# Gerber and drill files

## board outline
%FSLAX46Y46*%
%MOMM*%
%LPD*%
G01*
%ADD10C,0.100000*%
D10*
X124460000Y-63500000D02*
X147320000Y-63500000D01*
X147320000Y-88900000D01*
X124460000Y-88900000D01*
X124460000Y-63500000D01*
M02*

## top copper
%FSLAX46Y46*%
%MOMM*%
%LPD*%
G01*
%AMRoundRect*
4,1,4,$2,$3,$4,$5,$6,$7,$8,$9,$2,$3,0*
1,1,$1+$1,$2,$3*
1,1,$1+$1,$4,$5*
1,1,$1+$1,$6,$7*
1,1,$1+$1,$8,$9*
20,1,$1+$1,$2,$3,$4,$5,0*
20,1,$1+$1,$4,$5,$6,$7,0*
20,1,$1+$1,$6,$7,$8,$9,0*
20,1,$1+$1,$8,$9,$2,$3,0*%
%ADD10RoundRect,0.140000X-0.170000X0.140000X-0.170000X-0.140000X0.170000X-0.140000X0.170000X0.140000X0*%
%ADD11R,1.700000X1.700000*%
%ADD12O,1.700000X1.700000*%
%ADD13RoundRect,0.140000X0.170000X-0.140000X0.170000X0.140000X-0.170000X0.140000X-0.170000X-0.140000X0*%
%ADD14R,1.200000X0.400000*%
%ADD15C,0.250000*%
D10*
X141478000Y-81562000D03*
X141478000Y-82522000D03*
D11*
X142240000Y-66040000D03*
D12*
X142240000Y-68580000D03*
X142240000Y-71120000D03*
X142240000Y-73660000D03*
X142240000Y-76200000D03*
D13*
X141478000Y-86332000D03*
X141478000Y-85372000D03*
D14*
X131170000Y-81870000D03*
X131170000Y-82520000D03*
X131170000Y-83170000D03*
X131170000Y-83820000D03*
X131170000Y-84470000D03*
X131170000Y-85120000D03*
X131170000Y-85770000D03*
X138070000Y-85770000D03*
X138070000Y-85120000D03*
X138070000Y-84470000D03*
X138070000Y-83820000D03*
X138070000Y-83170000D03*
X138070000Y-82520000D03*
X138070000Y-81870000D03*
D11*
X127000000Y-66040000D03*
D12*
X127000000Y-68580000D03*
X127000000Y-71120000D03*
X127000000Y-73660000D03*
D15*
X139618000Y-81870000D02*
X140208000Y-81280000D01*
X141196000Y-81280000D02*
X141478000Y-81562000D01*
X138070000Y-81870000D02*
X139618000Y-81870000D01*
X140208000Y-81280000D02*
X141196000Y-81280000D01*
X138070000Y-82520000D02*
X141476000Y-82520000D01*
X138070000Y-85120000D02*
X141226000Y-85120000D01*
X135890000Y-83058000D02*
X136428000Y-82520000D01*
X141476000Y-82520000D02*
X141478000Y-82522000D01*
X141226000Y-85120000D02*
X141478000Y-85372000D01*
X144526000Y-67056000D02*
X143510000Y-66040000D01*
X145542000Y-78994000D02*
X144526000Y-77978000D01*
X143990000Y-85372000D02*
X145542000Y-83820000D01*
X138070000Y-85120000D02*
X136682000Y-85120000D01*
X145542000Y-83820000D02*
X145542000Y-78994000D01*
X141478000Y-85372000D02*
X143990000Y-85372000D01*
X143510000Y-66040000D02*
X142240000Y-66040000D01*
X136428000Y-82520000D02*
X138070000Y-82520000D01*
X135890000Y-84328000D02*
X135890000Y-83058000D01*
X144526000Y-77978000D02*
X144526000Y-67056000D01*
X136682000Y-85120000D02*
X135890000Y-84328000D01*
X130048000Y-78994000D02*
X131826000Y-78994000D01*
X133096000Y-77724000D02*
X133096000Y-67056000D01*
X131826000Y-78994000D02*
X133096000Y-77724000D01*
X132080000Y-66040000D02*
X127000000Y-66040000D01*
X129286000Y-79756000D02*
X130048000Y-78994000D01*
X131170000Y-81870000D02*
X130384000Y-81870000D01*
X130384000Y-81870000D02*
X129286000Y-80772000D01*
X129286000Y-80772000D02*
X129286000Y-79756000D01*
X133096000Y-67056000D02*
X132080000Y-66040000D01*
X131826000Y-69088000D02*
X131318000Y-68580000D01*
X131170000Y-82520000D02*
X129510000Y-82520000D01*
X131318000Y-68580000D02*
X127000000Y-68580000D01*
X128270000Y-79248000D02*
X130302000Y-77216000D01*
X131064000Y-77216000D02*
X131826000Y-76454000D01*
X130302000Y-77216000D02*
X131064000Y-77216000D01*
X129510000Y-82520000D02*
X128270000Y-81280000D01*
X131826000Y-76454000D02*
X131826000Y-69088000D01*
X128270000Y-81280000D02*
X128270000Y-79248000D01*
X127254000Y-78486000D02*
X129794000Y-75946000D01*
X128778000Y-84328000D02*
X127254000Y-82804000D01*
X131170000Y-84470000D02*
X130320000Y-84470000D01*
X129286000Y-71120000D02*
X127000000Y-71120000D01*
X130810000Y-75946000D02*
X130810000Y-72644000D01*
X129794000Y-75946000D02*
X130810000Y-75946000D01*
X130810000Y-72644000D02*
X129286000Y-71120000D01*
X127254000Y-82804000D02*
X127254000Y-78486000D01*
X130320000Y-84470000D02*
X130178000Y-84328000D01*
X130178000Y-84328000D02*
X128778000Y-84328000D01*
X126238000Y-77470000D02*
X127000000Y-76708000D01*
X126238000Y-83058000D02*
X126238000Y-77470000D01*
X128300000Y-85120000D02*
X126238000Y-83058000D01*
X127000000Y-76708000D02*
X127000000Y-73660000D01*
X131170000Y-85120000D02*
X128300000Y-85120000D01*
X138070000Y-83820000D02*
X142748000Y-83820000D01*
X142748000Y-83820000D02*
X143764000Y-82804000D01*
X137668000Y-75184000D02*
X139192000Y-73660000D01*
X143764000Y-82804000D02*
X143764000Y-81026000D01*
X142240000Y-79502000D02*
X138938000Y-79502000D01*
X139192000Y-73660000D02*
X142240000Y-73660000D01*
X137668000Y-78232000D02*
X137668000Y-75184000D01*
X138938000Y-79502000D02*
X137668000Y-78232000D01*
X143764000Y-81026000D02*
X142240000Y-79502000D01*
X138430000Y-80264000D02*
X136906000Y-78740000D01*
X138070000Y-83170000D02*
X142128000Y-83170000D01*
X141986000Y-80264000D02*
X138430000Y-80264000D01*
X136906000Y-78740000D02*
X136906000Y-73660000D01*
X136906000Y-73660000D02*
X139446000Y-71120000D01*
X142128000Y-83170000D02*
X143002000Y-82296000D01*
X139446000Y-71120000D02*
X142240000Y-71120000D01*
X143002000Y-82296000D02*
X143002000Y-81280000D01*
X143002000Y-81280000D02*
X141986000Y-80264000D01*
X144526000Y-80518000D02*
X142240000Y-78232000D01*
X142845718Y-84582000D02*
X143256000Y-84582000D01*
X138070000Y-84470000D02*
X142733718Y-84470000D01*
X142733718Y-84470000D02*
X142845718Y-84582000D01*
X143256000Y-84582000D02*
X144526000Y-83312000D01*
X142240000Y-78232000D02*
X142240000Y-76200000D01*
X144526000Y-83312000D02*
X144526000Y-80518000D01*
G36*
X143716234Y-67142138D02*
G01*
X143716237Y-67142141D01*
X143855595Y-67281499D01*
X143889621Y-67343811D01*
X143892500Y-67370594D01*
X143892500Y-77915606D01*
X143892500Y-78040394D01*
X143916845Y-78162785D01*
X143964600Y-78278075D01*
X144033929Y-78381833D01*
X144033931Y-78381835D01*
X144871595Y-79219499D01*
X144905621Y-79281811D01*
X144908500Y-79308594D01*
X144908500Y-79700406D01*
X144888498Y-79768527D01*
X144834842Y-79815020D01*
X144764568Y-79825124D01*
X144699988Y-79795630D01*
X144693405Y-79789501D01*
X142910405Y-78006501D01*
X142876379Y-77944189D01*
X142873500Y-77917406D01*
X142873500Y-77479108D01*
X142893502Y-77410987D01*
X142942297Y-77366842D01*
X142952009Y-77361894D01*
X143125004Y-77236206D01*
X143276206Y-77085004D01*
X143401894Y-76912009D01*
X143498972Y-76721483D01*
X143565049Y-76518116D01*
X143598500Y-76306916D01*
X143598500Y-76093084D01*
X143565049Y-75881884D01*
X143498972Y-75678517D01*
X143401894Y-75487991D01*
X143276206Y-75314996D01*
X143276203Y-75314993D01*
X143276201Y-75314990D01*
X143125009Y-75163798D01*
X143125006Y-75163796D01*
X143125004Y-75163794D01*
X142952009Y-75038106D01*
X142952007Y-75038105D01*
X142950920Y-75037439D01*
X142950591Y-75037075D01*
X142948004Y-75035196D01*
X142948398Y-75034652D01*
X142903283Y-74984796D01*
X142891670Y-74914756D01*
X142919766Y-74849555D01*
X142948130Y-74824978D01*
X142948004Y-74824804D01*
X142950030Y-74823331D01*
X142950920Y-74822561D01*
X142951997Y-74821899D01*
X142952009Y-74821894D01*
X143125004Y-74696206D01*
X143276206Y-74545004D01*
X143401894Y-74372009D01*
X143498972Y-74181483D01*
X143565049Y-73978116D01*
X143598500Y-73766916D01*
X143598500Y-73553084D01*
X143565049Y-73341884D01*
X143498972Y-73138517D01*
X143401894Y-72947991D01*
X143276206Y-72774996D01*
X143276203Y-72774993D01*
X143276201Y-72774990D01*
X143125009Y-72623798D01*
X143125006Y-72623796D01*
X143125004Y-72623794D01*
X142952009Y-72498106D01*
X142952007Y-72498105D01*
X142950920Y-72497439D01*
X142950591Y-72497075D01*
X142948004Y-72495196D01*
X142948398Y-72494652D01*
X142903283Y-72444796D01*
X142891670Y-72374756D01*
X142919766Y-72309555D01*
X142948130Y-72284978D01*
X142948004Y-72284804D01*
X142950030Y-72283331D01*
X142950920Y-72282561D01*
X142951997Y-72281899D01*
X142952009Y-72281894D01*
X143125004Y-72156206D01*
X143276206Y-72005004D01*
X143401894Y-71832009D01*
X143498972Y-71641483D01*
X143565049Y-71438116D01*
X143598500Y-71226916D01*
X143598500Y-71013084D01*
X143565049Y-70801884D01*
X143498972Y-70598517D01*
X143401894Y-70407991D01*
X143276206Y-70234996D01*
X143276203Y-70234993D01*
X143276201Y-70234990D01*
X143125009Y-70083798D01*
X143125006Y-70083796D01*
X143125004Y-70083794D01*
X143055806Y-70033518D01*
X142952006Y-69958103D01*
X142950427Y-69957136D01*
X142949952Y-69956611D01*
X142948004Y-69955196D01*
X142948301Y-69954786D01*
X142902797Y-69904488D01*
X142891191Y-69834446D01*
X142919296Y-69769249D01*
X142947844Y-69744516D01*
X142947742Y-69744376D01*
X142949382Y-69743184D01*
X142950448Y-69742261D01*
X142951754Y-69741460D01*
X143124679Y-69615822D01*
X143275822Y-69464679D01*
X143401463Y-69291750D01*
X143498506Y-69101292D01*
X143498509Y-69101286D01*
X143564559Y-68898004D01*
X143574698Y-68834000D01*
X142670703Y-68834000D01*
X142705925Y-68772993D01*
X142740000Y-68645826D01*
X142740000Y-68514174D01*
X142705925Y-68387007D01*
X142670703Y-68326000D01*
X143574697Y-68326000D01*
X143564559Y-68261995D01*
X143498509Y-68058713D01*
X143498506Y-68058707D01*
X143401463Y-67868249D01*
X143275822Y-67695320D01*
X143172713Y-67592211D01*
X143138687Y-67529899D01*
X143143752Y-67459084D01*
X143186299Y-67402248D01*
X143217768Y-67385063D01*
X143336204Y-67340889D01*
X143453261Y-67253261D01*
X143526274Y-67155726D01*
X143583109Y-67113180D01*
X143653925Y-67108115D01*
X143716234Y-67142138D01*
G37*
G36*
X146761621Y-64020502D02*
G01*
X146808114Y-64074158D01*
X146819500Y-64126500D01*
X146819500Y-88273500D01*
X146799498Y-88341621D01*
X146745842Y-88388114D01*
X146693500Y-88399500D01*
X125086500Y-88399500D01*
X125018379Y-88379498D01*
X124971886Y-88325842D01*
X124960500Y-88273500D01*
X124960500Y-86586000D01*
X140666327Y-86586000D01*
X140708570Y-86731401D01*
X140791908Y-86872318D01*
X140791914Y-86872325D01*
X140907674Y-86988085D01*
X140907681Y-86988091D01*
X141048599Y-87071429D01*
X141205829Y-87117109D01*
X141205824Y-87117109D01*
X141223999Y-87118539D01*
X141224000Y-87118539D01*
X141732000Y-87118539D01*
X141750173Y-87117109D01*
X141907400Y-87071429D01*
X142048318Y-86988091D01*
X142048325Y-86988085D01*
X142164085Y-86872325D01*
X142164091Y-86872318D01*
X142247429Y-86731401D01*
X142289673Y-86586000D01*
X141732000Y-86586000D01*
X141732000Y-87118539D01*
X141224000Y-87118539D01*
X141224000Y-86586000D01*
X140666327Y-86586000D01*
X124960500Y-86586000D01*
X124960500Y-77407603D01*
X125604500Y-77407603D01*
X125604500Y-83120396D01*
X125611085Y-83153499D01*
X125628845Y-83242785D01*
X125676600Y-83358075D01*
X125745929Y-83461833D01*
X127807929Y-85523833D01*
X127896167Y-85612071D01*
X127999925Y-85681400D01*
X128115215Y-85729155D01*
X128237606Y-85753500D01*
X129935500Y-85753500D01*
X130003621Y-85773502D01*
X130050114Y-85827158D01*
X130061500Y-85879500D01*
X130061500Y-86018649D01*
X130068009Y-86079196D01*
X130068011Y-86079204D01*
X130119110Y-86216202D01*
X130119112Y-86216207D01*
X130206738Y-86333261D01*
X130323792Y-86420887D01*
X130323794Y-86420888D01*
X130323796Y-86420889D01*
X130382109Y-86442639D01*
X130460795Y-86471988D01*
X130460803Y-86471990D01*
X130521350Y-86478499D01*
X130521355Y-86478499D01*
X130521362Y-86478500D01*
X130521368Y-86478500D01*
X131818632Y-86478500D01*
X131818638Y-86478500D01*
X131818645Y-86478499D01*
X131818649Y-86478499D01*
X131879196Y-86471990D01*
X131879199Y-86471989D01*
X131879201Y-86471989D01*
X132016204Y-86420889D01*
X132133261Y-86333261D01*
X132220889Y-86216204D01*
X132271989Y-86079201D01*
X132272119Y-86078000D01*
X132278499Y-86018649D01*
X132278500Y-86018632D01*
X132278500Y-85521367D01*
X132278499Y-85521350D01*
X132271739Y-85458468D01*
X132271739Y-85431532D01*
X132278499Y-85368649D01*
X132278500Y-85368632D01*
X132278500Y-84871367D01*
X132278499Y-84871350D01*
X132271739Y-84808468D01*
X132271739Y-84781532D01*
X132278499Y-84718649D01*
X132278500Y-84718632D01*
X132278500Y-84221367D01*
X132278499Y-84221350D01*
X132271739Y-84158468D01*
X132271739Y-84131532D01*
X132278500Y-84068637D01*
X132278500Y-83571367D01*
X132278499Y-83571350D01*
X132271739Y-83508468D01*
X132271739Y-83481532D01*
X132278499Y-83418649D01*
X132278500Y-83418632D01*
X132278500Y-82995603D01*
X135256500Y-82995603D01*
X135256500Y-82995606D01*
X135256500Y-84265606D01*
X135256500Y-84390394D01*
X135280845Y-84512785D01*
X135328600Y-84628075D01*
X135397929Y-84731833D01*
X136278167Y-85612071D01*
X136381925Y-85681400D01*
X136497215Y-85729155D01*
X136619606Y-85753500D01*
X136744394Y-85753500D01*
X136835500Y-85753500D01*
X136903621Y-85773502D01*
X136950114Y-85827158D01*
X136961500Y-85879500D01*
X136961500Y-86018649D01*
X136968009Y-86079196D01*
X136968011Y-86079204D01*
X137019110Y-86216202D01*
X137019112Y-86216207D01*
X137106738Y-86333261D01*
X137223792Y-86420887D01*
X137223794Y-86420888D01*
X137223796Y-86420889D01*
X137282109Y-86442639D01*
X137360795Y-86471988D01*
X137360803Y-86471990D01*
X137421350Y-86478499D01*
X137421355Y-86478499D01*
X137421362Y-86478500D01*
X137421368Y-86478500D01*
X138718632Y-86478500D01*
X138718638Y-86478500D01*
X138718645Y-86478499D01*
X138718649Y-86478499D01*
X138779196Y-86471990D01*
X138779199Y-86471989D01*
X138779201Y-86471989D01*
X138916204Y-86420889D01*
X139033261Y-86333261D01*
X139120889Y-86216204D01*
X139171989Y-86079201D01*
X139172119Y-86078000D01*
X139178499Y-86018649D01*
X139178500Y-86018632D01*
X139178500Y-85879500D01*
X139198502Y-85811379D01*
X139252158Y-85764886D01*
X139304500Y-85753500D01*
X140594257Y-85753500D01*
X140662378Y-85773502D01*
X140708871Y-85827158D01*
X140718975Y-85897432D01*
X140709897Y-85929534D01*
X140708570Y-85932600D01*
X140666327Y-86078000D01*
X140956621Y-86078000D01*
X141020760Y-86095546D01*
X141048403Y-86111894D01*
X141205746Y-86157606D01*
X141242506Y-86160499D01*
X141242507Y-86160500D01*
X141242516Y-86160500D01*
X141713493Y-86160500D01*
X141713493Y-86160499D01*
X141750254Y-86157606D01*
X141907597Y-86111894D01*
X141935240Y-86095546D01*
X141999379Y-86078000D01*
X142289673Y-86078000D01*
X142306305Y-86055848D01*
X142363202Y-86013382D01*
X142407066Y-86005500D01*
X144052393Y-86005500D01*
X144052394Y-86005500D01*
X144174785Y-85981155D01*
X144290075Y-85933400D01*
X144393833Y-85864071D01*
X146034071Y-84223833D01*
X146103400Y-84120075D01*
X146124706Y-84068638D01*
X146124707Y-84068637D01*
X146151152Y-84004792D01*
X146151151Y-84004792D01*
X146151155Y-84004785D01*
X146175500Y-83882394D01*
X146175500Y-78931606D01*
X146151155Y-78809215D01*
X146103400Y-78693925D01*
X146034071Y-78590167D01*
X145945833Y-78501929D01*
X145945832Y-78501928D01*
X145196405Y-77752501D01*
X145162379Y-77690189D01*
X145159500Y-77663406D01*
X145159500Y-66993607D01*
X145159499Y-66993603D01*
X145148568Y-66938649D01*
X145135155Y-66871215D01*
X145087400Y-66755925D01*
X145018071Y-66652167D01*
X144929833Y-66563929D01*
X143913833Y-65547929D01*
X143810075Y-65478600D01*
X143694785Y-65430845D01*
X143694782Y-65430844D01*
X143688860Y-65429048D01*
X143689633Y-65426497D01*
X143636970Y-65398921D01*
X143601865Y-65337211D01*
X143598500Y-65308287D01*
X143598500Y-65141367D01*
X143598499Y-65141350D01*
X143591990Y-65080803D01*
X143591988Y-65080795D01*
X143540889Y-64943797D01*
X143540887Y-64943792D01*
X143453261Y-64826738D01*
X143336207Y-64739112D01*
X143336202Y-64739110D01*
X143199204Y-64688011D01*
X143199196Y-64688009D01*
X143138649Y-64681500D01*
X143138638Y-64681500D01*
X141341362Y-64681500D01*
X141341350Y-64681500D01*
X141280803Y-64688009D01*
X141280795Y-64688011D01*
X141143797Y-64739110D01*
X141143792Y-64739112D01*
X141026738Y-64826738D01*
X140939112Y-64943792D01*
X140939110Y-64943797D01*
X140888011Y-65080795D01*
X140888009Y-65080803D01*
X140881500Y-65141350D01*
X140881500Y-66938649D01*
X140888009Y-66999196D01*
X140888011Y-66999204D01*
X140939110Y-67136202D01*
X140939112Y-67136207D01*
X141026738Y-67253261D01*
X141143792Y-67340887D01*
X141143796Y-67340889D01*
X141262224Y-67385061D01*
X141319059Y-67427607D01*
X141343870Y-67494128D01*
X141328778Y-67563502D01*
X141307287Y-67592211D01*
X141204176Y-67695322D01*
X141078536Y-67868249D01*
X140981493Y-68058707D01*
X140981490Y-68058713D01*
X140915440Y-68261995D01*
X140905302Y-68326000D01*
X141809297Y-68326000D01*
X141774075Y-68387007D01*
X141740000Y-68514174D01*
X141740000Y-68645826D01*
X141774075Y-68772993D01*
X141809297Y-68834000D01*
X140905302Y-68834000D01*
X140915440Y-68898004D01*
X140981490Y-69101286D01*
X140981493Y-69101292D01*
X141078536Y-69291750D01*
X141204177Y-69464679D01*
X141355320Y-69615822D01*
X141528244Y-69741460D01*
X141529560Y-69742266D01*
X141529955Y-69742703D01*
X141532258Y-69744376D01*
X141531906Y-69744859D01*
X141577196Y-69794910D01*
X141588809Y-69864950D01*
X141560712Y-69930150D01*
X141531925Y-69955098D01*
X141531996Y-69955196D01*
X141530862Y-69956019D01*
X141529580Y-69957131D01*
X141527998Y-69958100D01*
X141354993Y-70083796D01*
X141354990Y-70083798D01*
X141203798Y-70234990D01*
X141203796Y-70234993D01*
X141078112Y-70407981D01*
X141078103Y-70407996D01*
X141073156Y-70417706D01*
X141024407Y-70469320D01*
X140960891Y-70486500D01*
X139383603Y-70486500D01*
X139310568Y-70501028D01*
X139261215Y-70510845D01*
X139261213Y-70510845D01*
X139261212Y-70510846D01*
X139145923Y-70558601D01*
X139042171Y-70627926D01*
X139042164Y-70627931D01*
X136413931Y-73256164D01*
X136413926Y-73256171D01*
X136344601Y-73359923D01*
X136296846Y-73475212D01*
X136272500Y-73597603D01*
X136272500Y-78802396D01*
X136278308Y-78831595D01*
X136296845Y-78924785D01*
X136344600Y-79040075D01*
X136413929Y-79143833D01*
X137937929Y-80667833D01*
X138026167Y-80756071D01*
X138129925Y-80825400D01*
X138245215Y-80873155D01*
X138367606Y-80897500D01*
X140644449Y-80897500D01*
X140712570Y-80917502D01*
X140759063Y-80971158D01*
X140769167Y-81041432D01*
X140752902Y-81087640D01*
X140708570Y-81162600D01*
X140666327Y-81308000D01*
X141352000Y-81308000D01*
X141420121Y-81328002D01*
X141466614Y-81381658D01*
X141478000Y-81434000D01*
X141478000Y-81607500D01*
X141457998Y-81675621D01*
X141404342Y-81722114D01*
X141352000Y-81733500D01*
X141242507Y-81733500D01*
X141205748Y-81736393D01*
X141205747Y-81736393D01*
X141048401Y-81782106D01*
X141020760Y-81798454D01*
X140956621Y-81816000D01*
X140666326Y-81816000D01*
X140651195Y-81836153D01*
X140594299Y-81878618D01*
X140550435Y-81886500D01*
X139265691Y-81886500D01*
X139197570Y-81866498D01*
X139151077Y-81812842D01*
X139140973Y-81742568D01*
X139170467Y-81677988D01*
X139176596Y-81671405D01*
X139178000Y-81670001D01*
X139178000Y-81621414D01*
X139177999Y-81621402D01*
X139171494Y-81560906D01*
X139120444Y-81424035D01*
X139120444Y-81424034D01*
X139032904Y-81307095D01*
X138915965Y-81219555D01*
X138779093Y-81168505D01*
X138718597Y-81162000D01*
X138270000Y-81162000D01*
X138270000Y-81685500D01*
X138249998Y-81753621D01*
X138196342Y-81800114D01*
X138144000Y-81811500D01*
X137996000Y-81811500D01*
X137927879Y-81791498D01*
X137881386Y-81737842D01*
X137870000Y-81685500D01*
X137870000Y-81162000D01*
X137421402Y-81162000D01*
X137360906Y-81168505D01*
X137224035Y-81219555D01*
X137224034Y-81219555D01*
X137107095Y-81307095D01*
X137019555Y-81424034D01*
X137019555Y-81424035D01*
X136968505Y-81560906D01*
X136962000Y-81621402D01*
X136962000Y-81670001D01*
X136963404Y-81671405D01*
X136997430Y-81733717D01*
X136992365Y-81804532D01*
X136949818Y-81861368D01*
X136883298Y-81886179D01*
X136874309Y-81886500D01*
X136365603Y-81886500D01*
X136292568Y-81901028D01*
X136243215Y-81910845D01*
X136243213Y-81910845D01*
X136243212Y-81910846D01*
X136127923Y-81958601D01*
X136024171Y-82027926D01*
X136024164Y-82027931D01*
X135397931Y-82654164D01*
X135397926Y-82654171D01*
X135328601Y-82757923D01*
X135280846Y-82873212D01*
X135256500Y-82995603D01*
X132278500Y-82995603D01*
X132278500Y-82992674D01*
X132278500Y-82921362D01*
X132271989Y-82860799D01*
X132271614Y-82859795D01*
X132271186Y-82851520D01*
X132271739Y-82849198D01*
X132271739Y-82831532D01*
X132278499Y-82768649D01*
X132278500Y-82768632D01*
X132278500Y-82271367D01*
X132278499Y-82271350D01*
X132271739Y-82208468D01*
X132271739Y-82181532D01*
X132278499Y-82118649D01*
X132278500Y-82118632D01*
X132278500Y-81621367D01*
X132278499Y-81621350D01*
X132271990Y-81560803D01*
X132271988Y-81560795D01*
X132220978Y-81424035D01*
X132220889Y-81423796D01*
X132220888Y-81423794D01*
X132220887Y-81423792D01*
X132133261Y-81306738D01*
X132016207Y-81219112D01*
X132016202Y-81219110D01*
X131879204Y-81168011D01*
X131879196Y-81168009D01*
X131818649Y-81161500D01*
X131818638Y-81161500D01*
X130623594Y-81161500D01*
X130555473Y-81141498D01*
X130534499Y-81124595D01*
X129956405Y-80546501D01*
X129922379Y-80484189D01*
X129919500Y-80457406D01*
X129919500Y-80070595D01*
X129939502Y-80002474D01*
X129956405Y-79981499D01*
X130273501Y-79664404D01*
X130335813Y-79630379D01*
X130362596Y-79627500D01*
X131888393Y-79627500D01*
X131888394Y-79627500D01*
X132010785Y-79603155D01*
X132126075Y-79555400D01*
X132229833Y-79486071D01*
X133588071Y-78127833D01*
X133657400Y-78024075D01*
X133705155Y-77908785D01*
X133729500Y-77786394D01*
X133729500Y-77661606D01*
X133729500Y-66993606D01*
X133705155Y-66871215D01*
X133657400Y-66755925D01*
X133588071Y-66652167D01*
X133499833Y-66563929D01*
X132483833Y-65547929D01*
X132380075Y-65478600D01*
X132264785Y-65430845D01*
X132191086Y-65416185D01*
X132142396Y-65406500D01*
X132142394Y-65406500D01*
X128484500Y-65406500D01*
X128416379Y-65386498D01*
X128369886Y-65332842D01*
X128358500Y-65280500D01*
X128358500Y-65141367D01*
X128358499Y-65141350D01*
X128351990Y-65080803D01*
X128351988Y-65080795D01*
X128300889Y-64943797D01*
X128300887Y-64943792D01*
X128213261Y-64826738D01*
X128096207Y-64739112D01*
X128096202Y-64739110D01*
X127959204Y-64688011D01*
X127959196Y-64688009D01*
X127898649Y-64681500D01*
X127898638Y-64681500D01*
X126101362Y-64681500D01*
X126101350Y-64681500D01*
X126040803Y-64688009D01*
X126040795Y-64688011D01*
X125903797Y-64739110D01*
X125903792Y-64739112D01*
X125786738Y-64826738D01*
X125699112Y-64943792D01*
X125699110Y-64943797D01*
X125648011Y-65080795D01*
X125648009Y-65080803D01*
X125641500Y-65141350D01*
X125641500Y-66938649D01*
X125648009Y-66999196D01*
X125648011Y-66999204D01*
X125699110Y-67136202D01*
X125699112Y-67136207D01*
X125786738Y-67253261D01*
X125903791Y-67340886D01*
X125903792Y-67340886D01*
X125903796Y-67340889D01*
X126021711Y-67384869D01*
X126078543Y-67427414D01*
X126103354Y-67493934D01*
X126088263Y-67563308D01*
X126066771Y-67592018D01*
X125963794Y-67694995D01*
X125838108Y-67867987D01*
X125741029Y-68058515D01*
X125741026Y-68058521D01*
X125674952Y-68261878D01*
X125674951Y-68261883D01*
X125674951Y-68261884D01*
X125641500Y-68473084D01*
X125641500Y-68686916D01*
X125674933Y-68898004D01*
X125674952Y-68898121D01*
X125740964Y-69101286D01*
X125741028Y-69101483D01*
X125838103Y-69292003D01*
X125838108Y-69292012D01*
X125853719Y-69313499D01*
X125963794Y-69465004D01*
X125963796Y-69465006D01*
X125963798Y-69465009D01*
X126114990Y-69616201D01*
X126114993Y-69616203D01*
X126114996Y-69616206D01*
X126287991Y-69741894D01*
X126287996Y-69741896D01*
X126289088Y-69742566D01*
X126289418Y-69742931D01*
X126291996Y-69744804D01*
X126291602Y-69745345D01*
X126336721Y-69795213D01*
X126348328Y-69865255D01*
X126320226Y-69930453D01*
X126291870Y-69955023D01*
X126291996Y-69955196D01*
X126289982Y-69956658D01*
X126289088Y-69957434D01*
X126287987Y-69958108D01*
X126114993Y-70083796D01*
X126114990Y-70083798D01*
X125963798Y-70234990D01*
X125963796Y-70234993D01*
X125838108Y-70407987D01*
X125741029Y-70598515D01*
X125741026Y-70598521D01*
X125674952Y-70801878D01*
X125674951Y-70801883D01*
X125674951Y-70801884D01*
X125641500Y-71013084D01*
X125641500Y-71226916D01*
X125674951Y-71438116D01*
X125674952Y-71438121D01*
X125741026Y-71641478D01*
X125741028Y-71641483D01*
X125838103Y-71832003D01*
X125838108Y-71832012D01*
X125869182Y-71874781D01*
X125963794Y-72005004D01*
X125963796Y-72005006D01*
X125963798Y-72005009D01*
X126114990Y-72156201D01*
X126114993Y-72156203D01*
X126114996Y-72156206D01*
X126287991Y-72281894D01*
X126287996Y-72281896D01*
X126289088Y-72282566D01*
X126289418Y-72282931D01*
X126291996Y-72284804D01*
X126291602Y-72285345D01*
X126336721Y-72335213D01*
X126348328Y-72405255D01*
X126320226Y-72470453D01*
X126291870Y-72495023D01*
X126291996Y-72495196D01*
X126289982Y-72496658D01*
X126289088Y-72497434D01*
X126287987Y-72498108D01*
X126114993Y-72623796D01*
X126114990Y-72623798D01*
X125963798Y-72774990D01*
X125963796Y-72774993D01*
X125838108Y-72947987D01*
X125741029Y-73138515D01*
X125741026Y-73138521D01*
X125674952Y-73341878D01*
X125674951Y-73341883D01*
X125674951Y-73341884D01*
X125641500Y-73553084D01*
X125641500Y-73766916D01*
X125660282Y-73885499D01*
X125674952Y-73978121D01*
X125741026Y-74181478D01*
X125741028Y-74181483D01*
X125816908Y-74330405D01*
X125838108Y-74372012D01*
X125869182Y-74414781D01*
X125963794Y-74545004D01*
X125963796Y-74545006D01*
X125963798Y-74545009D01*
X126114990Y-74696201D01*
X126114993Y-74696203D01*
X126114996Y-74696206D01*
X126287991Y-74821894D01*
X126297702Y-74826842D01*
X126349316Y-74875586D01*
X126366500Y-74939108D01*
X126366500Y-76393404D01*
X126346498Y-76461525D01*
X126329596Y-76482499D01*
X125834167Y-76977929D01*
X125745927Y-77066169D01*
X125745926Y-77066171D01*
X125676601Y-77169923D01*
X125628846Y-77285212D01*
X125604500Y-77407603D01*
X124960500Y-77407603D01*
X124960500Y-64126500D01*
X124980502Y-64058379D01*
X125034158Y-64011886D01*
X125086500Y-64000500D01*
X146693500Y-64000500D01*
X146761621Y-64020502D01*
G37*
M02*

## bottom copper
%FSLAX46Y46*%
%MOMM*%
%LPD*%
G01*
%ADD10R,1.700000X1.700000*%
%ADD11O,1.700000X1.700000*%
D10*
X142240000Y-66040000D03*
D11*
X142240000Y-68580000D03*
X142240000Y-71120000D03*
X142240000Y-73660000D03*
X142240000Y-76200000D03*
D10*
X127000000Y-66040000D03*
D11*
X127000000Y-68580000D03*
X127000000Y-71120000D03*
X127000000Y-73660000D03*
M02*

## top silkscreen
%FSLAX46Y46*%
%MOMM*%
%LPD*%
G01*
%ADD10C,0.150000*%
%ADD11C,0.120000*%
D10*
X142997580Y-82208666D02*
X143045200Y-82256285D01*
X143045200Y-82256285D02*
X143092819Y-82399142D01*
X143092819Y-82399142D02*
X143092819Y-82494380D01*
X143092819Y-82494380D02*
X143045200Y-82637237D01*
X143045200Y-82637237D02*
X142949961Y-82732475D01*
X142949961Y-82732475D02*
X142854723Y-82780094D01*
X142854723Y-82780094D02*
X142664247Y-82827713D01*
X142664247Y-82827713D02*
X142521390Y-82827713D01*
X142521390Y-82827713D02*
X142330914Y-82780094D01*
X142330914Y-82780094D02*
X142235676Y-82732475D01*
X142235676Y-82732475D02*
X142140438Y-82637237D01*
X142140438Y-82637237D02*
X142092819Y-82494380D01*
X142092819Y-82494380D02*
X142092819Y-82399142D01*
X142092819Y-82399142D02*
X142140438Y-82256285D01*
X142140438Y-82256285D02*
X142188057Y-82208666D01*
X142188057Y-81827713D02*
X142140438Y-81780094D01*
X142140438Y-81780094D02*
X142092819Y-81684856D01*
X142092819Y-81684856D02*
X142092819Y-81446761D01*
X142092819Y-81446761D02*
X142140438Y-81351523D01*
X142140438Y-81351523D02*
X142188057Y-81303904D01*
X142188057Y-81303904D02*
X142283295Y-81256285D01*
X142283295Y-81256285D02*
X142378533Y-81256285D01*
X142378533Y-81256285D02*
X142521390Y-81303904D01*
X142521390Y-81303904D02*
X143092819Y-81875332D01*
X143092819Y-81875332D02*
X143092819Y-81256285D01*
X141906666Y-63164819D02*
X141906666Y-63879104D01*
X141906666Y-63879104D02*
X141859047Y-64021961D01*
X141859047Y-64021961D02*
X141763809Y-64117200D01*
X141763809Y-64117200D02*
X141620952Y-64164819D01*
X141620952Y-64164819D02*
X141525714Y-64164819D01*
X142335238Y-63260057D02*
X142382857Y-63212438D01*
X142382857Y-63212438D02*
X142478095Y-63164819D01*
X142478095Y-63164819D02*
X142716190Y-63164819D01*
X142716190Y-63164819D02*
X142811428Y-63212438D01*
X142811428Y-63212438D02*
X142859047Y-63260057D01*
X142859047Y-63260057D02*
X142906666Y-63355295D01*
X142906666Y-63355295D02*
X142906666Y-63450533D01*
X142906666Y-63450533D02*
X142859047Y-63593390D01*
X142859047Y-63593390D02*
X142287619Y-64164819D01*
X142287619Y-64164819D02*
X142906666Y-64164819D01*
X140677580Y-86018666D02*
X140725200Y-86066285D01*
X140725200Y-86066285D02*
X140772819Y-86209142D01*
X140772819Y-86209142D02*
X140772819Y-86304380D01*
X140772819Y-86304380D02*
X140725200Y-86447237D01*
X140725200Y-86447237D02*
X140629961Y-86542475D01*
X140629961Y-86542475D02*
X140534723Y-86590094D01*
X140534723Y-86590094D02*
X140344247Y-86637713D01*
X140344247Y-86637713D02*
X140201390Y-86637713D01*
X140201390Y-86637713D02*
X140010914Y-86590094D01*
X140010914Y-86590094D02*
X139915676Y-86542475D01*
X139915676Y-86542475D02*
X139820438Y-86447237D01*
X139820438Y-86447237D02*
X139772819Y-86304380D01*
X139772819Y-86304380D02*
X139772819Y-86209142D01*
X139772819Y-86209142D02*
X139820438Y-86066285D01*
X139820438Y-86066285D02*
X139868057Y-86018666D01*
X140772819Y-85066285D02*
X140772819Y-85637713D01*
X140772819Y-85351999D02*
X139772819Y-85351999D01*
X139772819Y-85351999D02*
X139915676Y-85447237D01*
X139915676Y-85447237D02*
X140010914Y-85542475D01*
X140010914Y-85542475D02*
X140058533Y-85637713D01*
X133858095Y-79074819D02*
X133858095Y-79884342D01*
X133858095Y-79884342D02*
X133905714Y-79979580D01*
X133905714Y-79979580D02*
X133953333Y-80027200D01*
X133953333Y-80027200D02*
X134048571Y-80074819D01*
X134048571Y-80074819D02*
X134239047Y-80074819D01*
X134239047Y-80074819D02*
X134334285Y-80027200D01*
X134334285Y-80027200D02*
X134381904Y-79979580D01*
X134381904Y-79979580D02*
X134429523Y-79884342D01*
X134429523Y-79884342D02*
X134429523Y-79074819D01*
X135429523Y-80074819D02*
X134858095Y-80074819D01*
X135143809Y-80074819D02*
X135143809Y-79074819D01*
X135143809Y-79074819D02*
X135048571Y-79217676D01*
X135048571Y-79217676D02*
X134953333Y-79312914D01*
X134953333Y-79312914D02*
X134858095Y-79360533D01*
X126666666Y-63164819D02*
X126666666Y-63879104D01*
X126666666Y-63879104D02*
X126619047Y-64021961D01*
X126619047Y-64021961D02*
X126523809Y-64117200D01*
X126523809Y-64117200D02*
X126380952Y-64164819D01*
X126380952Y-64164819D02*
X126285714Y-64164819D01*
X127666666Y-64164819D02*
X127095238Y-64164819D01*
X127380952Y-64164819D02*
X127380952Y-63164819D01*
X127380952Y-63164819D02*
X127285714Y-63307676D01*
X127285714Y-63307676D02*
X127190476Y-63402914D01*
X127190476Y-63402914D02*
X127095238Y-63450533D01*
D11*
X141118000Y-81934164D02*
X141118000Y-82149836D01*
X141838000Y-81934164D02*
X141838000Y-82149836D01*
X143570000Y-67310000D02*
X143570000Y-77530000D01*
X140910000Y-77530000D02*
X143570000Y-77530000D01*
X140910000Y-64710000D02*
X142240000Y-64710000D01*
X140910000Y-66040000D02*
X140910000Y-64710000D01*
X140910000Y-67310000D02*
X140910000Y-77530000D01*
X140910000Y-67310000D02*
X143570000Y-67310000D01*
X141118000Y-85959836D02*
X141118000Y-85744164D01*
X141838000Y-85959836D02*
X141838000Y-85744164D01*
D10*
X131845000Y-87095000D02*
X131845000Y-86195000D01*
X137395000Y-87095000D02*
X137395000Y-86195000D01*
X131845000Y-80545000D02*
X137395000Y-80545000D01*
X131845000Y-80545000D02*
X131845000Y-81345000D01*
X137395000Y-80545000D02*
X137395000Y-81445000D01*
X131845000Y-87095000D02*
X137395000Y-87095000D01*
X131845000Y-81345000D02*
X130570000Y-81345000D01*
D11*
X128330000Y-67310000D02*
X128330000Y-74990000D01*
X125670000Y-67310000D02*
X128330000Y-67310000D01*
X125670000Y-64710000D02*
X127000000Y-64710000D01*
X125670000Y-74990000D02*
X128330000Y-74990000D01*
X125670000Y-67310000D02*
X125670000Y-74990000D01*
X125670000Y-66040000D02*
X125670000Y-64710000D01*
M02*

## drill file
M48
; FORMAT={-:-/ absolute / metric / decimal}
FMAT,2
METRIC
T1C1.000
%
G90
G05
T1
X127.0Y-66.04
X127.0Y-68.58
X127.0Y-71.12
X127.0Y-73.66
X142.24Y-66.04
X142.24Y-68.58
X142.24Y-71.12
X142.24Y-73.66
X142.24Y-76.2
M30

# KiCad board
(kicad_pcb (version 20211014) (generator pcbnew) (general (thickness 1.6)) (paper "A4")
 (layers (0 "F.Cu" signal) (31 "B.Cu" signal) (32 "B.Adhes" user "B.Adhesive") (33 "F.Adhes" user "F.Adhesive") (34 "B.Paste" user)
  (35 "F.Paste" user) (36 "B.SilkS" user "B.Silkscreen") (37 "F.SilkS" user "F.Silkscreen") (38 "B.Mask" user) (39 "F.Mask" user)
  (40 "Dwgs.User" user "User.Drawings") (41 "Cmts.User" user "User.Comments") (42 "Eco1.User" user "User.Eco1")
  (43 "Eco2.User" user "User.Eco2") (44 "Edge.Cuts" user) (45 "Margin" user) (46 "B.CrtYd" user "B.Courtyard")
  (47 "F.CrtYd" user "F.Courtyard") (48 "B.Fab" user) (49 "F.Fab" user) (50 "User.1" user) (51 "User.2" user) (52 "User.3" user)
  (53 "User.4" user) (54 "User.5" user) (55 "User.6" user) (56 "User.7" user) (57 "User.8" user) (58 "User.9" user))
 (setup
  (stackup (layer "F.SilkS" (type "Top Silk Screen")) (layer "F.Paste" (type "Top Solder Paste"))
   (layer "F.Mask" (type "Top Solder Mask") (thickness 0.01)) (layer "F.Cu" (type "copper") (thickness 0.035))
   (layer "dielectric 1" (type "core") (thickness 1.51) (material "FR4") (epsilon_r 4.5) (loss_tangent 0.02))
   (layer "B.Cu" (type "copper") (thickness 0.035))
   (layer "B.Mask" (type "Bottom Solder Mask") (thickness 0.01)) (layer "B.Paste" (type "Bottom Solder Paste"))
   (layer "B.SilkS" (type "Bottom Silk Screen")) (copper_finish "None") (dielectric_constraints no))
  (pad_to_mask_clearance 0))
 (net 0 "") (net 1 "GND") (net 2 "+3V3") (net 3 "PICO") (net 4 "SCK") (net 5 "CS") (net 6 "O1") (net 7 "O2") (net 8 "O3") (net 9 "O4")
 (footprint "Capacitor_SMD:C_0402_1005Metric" (layer "F.Cu") (at 141.478 82.042 -90)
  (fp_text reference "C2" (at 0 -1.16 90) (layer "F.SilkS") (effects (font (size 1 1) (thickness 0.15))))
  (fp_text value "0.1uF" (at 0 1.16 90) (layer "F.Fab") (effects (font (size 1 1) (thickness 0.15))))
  (fp_line (start -0.107836 0.36) (end 0.107836 0.36) (layer "F.SilkS") (width 0.12))
  (fp_line (start -0.107836 -0.36) (end 0.107836 -0.36) (layer "F.SilkS") (width 0.12))
  (pad "1" smd roundrect (at -0.48 0 270) (size 0.56 0.62) (layers "F.Cu" "F.Paste" "F.Mask") (roundrect_rratio 0.25) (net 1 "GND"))
  (pad "2" smd roundrect (at 0.48 0 270) (size 0.56 0.62) (layers "F.Cu" "F.Paste" "F.Mask") (roundrect_rratio 0.25) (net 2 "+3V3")))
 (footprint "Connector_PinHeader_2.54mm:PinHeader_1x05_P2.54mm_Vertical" (layer "F.Cu") (at 142.24 66.04)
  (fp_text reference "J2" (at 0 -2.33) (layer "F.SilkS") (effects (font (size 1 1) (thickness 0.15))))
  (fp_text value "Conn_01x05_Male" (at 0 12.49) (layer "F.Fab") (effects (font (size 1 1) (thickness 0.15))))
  (fp_line (start 1.33 1.27) (end 1.33 11.49) (layer "F.SilkS") (width 0.12))
  (fp_line (start -1.33 11.49) (end 1.33 11.49) (layer "F.SilkS") (width 0.12))
  (fp_line (start -1.33 -1.33) (end 0 -1.33) (layer "F.SilkS") (width 0.12))
  (fp_line (start -1.33 0) (end -1.33 -1.33) (layer "F.SilkS") (width 0.12))
  (fp_line (start -1.33 1.27) (end -1.33 11.49) (layer "F.SilkS") (width 0.12))
  (fp_line (start -1.33 1.27) (end 1.33 1.27) (layer "F.SilkS") (width 0.12))
  (pad "1" thru_hole rect (at 0 0) (size 1.7 1.7) (drill 1) (layers *.Cu *.Mask) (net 2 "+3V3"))
  (pad "2" thru_hole oval (at 0 2.54) (size 1.7 1.7) (drill 1) (layers *.Cu *.Mask) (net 1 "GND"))
  (pad "3" thru_hole oval (at 0 5.08) (size 1.7 1.7) (drill 1) (layers *.Cu *.Mask) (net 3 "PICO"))
  (pad "4" thru_hole oval (at 0 7.62) (size 1.7 1.7) (drill 1) (layers *.Cu *.Mask) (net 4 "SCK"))
  (pad "5" thru_hole oval (at 0 10.16) (size 1.7 1.7) (drill 1) (layers *.Cu *.Mask) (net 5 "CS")))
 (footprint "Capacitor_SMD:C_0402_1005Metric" (layer "F.Cu") (at 141.478 85.852 90)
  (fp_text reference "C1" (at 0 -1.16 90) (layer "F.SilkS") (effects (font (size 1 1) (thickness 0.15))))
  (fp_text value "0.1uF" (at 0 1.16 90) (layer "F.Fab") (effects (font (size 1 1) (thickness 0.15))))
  (fp_line (start -0.107836 -0.36) (end 0.107836 -0.36) (layer "F.SilkS") (width 0.12))
  (fp_line (start -0.107836 0.36) (end 0.107836 0.36) (layer "F.SilkS") (width 0.12))
  (pad "1" smd roundrect (at -0.48 0 90) (size 0.56 0.62) (layers "F.Cu" "F.Paste" "F.Mask") (roundrect_rratio 0.25) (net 1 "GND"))
  (pad "2" smd roundrect (at 0.48 0 90) (size 0.56 0.62) (layers "F.Cu" "F.Paste" "F.Mask") (roundrect_rratio 0.25) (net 2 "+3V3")))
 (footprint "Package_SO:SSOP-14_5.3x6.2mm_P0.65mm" (layer "F.Cu") (at 134.62 83.82)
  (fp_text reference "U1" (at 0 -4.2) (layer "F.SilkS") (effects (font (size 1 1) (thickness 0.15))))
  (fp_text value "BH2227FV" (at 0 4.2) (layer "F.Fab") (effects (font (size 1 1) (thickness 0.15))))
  (fp_line (start -2.775 3.275) (end -2.775 2.375) (layer "F.SilkS") (width 0.15))
  (fp_line (start 2.775 3.275) (end 2.775 2.375) (layer "F.SilkS") (width 0.15))
  (fp_line (start -2.775 -3.275) (end 2.775 -3.275) (layer "F.SilkS") (width 0.15))
  (fp_line (start -2.775 -3.275) (end -2.775 -2.475) (layer "F.SilkS") (width 0.15))
  (fp_line (start 2.775 -3.275) (end 2.775 -2.375) (layer "F.SilkS") (width 0.15))
  (fp_line (start -2.775 3.275) (end 2.775 3.275) (layer "F.SilkS") (width 0.15))
  (fp_line (start -2.775 -2.475) (end -4.05 -2.475) (layer "F.SilkS") (width 0.15))
  (pad "1" smd rect (at -3.45 -1.95) (size 1.2 0.4) (layers "F.Cu" "F.Paste" "F.Mask") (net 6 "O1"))
  (pad "2" smd rect (at -3.45 -1.3) (size 1.2 0.4) (layers "F.Cu" "F.Paste" "F.Mask") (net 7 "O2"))
  (pad "3" smd rect (at -3.45 -0.65) (size 1.2 0.4) (layers "F.Cu" "F.Paste" "F.Mask"))
  (pad "4" smd rect (at -3.45 0) (size 1.2 0.4) (layers "F.Cu" "F.Paste" "F.Mask"))
  (pad "5" smd rect (at -3.45 0.65) (size 1.2 0.4) (layers "F.Cu" "F.Paste" "F.Mask") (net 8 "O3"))
  (pad "6" smd rect (at -3.45 1.3) (size 1.2 0.4) (layers "F.Cu" "F.Paste" "F.Mask") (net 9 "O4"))
  (pad "7" smd rect (at -3.45 1.95) (size 1.2 0.4) (layers "F.Cu" "F.Paste" "F.Mask"))
  (pad "8" smd rect (at 3.45 1.95) (size 1.2 0.4) (layers "F.Cu" "F.Paste" "F.Mask"))
  (pad "9" smd rect (at 3.45 1.3) (size 1.2 0.4) (layers "F.Cu" "F.Paste" "F.Mask") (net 2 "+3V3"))
  (pad "10" smd rect (at 3.45 0.65) (size 1.2 0.4) (layers "F.Cu" "F.Paste" "F.Mask") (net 5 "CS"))
  (pad "11" smd rect (at 3.45 0) (size 1.2 0.4) (layers "F.Cu" "F.Paste" "F.Mask") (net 4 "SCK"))
  (pad "12" smd rect (at 3.45 -0.65) (size 1.2 0.4) (layers "F.Cu" "F.Paste" "F.Mask") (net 3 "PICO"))
  (pad "13" smd rect (at 3.45 -1.3) (size 1.2 0.4) (layers "F.Cu" "F.Paste" "F.Mask") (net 2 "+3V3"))
  (pad "14" smd rect (at 3.45 -1.95) (size 1.2 0.4) (layers "F.Cu" "F.Paste" "F.Mask") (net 1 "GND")))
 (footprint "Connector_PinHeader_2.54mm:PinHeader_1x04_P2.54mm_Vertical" (layer "F.Cu") (at 127 66.04)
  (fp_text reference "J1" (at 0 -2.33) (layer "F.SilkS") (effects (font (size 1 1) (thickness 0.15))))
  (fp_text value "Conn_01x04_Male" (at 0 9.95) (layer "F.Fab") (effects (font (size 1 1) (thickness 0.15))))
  (fp_line (start 1.33 1.27) (end 1.33 8.95) (layer "F.SilkS") (width 0.12))
  (fp_line (start -1.33 1.27) (end 1.33 1.27) (layer "F.SilkS") (width 0.12))
  (fp_line (start -1.33 -1.33) (end 0 -1.33) (layer "F.SilkS") (width 0.12))
  (fp_line (start -1.33 8.95) (end 1.33 8.95) (layer "F.SilkS") (width 0.12))
  (fp_line (start -1.33 1.27) (end -1.33 8.95) (layer "F.SilkS") (width 0.12))
  (fp_line (start -1.33 0) (end -1.33 -1.33) (layer "F.SilkS") (width 0.12))
  (pad "1" thru_hole rect (at 0 0) (size 1.7 1.7) (drill 1) (layers *.Cu *.Mask) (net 6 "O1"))
  (pad "2" thru_hole oval (at 0 2.54) (size 1.7 1.7) (drill 1) (layers *.Cu *.Mask) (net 7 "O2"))
  (pad "3" thru_hole oval (at 0 5.08) (size 1.7 1.7) (drill 1) (layers *.Cu *.Mask) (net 8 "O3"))
  (pad "4" thru_hole oval (at 0 7.62) (size 1.7 1.7) (drill 1) (layers *.Cu *.Mask) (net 9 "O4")))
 (gr_rect (start 124.46 63.5) (end 147.32 88.9) (layer "Edge.Cuts") (width 0.1) (fill none))
 (segment (start 139.618 81.87) (end 140.208 81.28) (width 0.25) (layer "F.Cu") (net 1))
 (segment (start 141.196 81.28) (end 141.478 81.562) (width 0.25) (layer "F.Cu") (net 1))
 (segment (start 138.07 81.87) (end 139.618 81.87) (width 0.25) (layer "F.Cu") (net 1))
 (segment (start 140.208 81.28) (end 141.196 81.28) (width 0.25) (layer "F.Cu") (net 1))
 (segment (start 138.07 82.52) (end 141.476 82.52) (width 0.25) (layer "F.Cu") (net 2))
 (segment (start 138.07 85.12) (end 141.226 85.12) (width 0.25) (layer "F.Cu") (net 2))
 (segment (start 135.89 83.058) (end 136.428 82.52) (width 0.25) (layer "F.Cu") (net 2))
 (segment (start 141.476 82.52) (end 141.478 82.522) (width 0.25) (layer "F.Cu") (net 2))
 (segment (start 141.226 85.12) (end 141.478 85.372) (width 0.25) (layer "F.Cu") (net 2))
 (segment (start 144.526 67.056) (end 143.51 66.04) (width 0.25) (layer "F.Cu") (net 2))
 (segment (start 145.542 78.994) (end 144.526 77.978) (width 0.25) (layer "F.Cu") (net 2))
 (segment (start 143.99 85.372) (end 145.542 83.82) (width 0.25) (layer "F.Cu") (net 2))
 (segment (start 138.07 85.12) (end 136.682 85.12) (width 0.25) (layer "F.Cu") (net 2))
 (segment (start 145.542 83.82) (end 145.542 78.994) (width 0.25) (layer "F.Cu") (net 2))
 (segment (start 141.478 85.372) (end 143.99 85.372) (width 0.25) (layer "F.Cu") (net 2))
 (segment (start 143.51 66.04) (end 142.24 66.04) (width 0.25) (layer "F.Cu") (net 2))
 (segment (start 136.428 82.52) (end 138.07 82.52) (width 0.25) (layer "F.Cu") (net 2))
 (segment (start 135.89 84.328) (end 135.89 83.058) (width 0.25) (layer "F.Cu") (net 2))
 (segment (start 144.526 77.978) (end 144.526 67.056) (width 0.25) (layer "F.Cu") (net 2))
 (segment (start 136.682 85.12) (end 135.89 84.328) (width 0.25) (layer "F.Cu") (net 2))
 (segment (start 130.048 78.994) (end 131.826 78.994) (width 0.25) (layer "F.Cu") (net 6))
 (segment (start 133.096 77.724) (end 133.096 67.056) (width 0.25) (layer "F.Cu") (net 6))
 (segment (start 131.826 78.994) (end 133.096 77.724) (width 0.25) (layer "F.Cu") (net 6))
 (segment (start 132.08 66.04) (end 127 66.04) (width 0.25) (layer "F.Cu") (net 6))
 (segment (start 129.286 79.756) (end 130.048 78.994) (width 0.25) (layer "F.Cu") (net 6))
 (segment (start 131.17 81.87) (end 130.384 81.87) (width 0.25) (layer "F.Cu") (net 6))
 (segment (start 130.384 81.87) (end 129.286 80.772) (width 0.25) (layer "F.Cu") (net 6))
 (segment (start 129.286 80.772) (end 129.286 79.756) (width 0.25) (layer "F.Cu") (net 6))
 (segment (start 133.096 67.056) (end 132.08 66.04) (width 0.25) (layer "F.Cu") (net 6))
 (segment (start 131.826 69.088) (end 131.318 68.58) (width 0.25) (layer "F.Cu") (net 7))
 (segment (start 131.17 82.52) (end 129.51 82.52) (width 0.25) (layer "F.Cu") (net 7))
 (segment (start 131.318 68.58) (end 127 68.58) (width 0.25) (layer "F.Cu") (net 7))
 (segment (start 128.27 79.248) (end 130.302 77.216) (width 0.25) (layer "F.Cu") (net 7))
 (segment (start 131.064 77.216) (end 131.826 76.454) (width 0.25) (layer "F.Cu") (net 7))
 (segment (start 130.302 77.216) (end 131.064 77.216) (width 0.25) (layer "F.Cu") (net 7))
 (segment (start 129.51 82.52) (end 128.27 81.28) (width 0.25) (layer "F.Cu") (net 7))
 (segment (start 131.826 76.454) (end 131.826 69.088) (width 0.25) (layer "F.Cu") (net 7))
 (segment (start 128.27 81.28) (end 128.27 79.248) (width 0.25) (layer "F.Cu") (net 7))
 (segment (start 127.254 78.486) (end 129.794 75.946) (width 0.25) (layer "F.Cu") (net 8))
 (segment (start 128.778 84.328) (end 127.254 82.804) (width 0.25) (layer "F.Cu") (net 8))
 (segment (start 131.17 84.47) (end 130.32 84.47) (width 0.25) (layer "F.Cu") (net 8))
 (segment (start 129.286 71.12) (end 127 71.12) (width 0.25) (layer "F.Cu") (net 8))
 (segment (start 130.81 75.946) (end 130.81 72.644) (width 0.25) (layer "F.Cu") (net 8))
 (segment (start 129.794 75.946) (end 130.81 75.946) (width 0.25) (layer "F.Cu") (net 8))
 (segment (start 130.81 72.644) (end 129.286 71.12) (width 0.25) (layer "F.Cu") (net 8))
 (segment (start 127.254 82.804) (end 127.254 78.486) (width 0.25) (layer "F.Cu") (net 8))
 (segment (start 130.32 84.47) (end 130.178 84.328) (width 0.25) (layer "F.Cu") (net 8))
 (segment (start 130.178 84.328) (end 128.778 84.328) (width 0.25) (layer "F.Cu") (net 8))
 (segment (start 126.238 77.47) (end 127 76.708) (width 0.25) (layer "F.Cu") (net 9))
 (segment (start 126.238 83.058) (end 126.238 77.47) (width 0.25) (layer "F.Cu") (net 9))
 (segment (start 128.3 85.12) (end 126.238 83.058) (width 0.25) (layer "F.Cu") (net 9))
 (segment (start 127 76.708) (end 127 73.66) (width 0.25) (layer "F.Cu") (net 9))
 (segment (start 131.17 85.12) (end 128.3 85.12) (width 0.25) (layer "F.Cu") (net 9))
 (segment (start 138.07 83.82) (end 142.748 83.82) (width 0.25) (layer "F.Cu") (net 4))
 (segment (start 142.748 83.82) (end 143.764 82.804) (width 0.25) (layer "F.Cu") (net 4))
 (segment (start 137.668 75.184) (end 139.192 73.66) (width 0.25) (layer "F.Cu") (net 4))
 (segment (start 143.764 82.804) (end 143.764 81.026) (width 0.25) (layer "F.Cu") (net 4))
 (segment (start 142.24 79.502) (end 138.938 79.502) (width 0.25) (layer "F.Cu") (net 4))
 (segment (start 139.192 73.66) (end 142.24 73.66) (width 0.25) (layer "F.Cu") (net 4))
 (segment (start 137.668 78.232) (end 137.668 75.184) (width 0.25) (layer "F.Cu") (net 4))
 (segment (start 138.938 79.502) (end 137.668 78.232) (width 0.25) (layer "F.Cu") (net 4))
 (segment (start 143.764 81.026) (end 142.24 79.502) (width 0.25) (layer "F.Cu") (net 4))
 (segment (start 138.43 80.264) (end 136.906 78.74) (width 0.25) (layer "F.Cu") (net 3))
 (segment (start 138.07 83.17) (end 142.128 83.17) (width 0.25) (layer "F.Cu") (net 3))
 (segment (start 141.986 80.264) (end 138.43 80.264) (width 0.25) (layer "F.Cu") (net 3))
 (segment (start 136.906 78.74) (end 136.906 73.66) (width 0.25) (layer "F.Cu") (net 3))
 (segment (start 136.906 73.66) (end 139.446 71.12) (width 0.25) (layer "F.Cu") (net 3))
 (segment (start 142.128 83.17) (end 143.002 82.296) (width 0.25) (layer "F.Cu") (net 3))
 (segment (start 139.446 71.12) (end 142.24 71.12) (width 0.25) (layer "F.Cu") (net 3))
 (segment (start 143.002 82.296) (end 143.002 81.28) (width 0.25) (layer "F.Cu") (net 3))
 (segment (start 143.002 81.28) (end 141.986 80.264) (width 0.25) (layer "F.Cu") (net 3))
 (segment (start 144.526 80.518) (end 142.24 78.232) (width 0.25) (layer "F.Cu") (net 5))
 (segment (start 142.845718 84.582) (end 143.256 84.582) (width 0.25) (layer "F.Cu") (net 5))
 (segment (start 138.07 84.47) (end 142.733718 84.47) (width 0.25) (layer "F.Cu") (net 5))
 (segment (start 142.733718 84.47) (end 142.845718 84.582) (width 0.25) (layer "F.Cu") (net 5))
 (segment (start 143.256 84.582) (end 144.526 83.312) (width 0.25) (layer "F.Cu") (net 5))
 (segment (start 142.24 78.232) (end 142.24 76.2) (width 0.25) (layer "F.Cu") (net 5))
 (segment (start 144.526 83.312) (end 144.526 80.518) (width 0.25) (layer "F.Cu") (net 5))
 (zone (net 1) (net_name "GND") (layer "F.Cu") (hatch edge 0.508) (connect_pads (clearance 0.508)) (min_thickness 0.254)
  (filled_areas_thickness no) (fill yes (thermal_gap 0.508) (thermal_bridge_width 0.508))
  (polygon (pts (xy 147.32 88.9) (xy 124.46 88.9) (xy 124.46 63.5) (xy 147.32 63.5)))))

